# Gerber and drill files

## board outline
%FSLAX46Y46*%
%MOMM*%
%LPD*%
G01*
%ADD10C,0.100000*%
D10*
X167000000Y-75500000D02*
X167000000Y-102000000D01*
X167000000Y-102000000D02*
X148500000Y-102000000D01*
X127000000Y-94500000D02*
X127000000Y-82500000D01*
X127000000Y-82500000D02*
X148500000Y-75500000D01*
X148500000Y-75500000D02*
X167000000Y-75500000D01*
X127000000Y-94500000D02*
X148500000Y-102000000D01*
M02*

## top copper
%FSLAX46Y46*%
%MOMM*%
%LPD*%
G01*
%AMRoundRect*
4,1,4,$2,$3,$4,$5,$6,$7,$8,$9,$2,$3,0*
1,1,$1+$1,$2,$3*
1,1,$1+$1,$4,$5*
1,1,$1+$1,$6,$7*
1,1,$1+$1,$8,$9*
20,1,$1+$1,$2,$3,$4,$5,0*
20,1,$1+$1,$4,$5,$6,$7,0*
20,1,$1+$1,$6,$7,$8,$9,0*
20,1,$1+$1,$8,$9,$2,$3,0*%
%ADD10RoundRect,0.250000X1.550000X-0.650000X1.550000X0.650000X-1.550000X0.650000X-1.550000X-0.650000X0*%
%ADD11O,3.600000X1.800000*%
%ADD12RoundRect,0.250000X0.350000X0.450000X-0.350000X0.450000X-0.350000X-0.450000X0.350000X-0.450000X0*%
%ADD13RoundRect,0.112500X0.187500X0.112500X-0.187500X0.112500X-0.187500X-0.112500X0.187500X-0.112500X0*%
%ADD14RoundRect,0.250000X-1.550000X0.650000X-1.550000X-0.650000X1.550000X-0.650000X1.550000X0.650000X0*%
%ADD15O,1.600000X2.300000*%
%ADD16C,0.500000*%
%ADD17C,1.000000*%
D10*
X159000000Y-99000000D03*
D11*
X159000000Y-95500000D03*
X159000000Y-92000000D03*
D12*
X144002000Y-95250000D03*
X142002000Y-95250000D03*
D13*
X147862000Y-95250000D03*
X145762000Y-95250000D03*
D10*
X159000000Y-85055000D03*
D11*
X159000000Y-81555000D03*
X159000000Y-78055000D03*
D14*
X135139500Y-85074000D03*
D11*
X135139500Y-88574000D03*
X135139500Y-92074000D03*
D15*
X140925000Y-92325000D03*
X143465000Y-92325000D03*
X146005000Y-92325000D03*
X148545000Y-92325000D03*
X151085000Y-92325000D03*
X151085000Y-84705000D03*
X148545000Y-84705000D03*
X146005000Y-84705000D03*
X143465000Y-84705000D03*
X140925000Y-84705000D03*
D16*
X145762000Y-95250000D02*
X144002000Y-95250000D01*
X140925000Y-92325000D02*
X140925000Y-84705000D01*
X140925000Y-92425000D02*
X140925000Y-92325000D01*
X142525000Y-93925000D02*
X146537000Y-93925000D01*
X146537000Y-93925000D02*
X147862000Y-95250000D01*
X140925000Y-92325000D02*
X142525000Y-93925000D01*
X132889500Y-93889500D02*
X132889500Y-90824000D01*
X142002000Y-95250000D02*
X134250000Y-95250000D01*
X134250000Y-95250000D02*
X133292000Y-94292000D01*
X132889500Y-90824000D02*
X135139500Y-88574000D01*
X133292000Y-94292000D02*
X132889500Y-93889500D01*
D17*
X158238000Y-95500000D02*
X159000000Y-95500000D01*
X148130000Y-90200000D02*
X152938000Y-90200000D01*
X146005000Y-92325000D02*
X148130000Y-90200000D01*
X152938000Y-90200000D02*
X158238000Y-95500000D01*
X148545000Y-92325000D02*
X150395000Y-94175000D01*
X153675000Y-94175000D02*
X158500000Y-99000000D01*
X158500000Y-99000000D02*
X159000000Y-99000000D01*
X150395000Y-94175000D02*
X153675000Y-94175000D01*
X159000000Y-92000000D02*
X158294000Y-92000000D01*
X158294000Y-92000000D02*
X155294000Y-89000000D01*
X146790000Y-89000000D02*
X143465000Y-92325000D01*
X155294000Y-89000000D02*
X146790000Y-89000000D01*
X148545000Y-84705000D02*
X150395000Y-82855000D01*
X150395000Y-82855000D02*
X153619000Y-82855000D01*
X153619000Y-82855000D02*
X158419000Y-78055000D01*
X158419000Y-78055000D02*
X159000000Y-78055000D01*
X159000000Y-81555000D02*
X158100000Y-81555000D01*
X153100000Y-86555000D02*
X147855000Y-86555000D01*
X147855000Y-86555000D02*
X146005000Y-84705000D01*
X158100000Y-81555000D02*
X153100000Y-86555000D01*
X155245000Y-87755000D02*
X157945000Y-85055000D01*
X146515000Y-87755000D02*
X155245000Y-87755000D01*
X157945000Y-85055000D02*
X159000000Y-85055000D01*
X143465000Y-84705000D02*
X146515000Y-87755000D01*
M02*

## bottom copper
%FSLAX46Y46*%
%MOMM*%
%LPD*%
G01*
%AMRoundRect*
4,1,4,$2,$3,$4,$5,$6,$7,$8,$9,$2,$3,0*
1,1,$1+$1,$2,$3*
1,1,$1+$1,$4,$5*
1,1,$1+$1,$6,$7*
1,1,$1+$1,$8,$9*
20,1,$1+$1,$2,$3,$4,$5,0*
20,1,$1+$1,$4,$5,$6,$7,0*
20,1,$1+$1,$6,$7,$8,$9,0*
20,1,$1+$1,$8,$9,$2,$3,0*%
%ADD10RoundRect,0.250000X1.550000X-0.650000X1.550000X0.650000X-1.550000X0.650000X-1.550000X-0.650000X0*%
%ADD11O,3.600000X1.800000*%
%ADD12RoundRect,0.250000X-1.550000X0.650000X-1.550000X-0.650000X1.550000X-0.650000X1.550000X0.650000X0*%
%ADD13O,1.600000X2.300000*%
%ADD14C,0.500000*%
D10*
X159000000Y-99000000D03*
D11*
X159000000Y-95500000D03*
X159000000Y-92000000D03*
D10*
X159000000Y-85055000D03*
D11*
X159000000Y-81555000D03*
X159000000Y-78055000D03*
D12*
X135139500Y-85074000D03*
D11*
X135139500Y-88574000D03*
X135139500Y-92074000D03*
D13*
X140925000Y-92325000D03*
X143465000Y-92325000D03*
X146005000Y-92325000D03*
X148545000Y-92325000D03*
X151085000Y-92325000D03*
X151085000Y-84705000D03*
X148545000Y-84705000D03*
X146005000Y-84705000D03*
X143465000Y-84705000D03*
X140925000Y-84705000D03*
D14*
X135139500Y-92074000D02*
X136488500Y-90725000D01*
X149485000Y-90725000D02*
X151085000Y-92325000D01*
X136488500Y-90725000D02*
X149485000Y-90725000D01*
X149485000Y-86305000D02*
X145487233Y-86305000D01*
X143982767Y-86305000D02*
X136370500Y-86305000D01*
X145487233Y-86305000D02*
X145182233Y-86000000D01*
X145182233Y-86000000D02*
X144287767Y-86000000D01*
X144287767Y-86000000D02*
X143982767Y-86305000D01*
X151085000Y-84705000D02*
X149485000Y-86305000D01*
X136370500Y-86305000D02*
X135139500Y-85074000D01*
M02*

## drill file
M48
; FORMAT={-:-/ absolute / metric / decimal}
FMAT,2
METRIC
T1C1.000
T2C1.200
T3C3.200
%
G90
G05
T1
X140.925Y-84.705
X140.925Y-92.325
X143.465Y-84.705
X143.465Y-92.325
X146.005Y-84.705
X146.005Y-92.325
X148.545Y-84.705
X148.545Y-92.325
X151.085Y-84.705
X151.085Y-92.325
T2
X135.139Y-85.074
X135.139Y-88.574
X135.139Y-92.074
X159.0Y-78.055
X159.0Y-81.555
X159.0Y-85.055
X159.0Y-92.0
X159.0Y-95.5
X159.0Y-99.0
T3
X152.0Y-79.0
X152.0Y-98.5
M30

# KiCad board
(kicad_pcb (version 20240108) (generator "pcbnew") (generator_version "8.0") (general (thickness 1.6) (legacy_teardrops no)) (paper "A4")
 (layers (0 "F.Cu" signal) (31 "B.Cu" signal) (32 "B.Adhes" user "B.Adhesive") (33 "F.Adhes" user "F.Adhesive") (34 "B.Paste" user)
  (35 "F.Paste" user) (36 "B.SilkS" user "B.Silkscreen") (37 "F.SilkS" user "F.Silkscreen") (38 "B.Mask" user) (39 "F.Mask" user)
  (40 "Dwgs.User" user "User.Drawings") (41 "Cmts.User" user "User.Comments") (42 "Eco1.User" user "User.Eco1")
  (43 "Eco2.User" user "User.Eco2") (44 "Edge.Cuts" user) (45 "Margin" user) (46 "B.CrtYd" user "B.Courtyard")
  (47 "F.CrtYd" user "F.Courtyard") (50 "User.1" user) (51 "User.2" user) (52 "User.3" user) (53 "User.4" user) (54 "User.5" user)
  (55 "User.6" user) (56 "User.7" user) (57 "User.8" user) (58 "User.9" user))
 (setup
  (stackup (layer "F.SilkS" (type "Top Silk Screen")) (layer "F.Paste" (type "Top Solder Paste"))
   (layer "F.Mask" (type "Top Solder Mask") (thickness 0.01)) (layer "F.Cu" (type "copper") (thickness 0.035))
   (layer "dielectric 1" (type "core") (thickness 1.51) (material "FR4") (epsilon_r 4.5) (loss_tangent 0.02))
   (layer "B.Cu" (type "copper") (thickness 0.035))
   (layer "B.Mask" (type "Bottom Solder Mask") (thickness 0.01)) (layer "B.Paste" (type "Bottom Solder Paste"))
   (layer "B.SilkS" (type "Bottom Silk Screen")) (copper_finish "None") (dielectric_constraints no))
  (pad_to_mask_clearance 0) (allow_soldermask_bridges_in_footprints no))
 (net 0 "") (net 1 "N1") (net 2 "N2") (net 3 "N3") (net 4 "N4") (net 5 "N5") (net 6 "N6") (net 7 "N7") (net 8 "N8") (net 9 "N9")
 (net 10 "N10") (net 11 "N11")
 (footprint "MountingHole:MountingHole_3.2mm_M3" (layer "F.Cu") (at 152 98.5)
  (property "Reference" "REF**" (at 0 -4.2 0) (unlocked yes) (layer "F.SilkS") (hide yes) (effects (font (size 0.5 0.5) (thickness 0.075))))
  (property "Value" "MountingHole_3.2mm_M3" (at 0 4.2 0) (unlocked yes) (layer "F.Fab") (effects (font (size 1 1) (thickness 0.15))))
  (pad "" np_thru_hole circle (at 0 0) (size 3.2 3.2) (drill 3.2) (layers "*.Cu" "*.Mask")))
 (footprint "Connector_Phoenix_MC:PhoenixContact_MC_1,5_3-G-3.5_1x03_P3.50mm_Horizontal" (layer "F.Cu") (at 159 99 90)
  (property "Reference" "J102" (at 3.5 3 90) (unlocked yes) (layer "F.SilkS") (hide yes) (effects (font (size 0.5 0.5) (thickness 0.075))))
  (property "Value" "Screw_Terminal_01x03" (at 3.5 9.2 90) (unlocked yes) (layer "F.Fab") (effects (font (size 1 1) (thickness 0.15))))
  (pad "1" thru_hole roundrect (at 0 0 90) (size 1.8 3.6) (drill 1.2) (layers "*.Cu" "*.Mask") (remove_unused_layers no)
   (roundrect_rratio 0.138889) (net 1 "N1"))
  (pad "2" thru_hole oval (at 3.5 0 90) (size 1.8 3.6) (drill 1.2) (layers "*.Cu" "*.Mask") (remove_unused_layers no) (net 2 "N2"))
  (pad "3" thru_hole oval (at 7 0 90) (size 1.8 3.6) (drill 1.2) (layers "*.Cu" "*.Mask") (remove_unused_layers no) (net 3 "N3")))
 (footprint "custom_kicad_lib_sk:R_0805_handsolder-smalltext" (layer "F.Cu") (at 143.002 95.25 180)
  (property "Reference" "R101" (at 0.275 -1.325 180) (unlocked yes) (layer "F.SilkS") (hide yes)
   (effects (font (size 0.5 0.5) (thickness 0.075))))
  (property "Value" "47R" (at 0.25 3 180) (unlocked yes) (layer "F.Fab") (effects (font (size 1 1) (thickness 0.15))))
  (pad "1" smd roundrect (at -1 0 180) (size 1.2 1.4) (layers "F.Cu" "F.Paste" "F.Mask") (roundrect_rratio 0.208333) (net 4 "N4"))
  (pad "2" smd roundrect (at 1 0 180) (size 1.2 1.4) (layers "F.Cu" "F.Paste" "F.Mask") (roundrect_rratio 0.208333) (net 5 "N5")))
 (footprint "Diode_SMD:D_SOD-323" (layer "F.Cu") (at 146.812 95.25 180)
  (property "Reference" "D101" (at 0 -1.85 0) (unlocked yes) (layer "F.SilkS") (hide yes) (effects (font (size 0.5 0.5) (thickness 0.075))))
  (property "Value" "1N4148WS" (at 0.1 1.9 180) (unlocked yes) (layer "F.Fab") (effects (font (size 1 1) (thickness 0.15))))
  (pad "1" smd roundrect (at -1.05 0 180) (size 0.6 0.45) (layers "F.Cu" "F.Paste" "F.Mask") (roundrect_rratio 0.25) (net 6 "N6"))
  (pad "2" smd roundrect (at 1.05 0 180) (size 0.6 0.45) (layers "F.Cu" "F.Paste" "F.Mask") (roundrect_rratio 0.25) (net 4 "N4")))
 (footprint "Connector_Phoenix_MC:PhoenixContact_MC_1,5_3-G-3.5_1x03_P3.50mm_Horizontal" (layer "F.Cu") (at 159 85.055 90)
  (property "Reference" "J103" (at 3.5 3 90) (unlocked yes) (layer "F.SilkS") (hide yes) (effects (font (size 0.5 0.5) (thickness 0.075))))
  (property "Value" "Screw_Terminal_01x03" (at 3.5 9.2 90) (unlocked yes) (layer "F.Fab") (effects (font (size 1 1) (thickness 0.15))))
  (pad "1" thru_hole roundrect (at 0 0 90) (size 1.8 3.6) (drill 1.2) (layers "*.Cu" "*.Mask") (remove_unused_layers no)
   (roundrect_rratio 0.138889) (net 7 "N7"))
  (pad "2" thru_hole oval (at 3.5 0 90) (size 1.8 3.6) (drill 1.2) (layers "*.Cu" "*.Mask") (remove_unused_layers no) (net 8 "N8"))
  (pad "3" thru_hole oval (at 7 0 90) (size 1.8 3.6) (drill 1.2) (layers "*.Cu" "*.Mask") (remove_unused_layers no) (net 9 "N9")))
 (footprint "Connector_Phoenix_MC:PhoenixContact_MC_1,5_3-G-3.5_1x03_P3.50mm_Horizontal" (layer "F.Cu") (at 135.1395 85.074 -90)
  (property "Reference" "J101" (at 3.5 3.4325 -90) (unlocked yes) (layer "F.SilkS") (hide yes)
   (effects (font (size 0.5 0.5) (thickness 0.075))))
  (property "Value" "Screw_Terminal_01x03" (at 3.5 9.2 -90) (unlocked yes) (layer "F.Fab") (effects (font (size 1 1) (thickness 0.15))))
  (pad "1" thru_hole roundrect (at 0 0 270) (size 1.8 3.6) (drill 1.2) (layers "*.Cu" "*.Mask") (remove_unused_layers no)
   (roundrect_rratio 0.138889) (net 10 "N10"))
  (pad "2" thru_hole oval (at 3.5 0 270) (size 1.8 3.6) (drill 1.2) (layers "*.Cu" "*.Mask") (remove_unused_layers no) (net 5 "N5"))
  (pad "3" thru_hole oval (at 7 0 270) (size 1.8 3.6) (drill 1.2) (layers "*.Cu" "*.Mask") (remove_unused_layers no) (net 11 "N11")))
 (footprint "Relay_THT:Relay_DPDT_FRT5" (layer "F.Cu") (at 140.925 92.325 90)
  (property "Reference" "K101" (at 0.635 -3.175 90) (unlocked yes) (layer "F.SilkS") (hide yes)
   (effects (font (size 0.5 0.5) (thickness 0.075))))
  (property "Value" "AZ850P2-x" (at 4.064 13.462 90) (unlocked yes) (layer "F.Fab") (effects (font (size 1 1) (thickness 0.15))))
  (pad "1" thru_hole oval (at 0 0 90) (size 2.3 1.6) (drill 1) (layers "*.Cu" "*.Mask") (remove_unused_layers no) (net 6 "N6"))
  (pad "2" thru_hole oval (at 0 2.54 90) (size 2.3 1.6) (drill 1) (layers "*.Cu" "*.Mask") (remove_unused_layers no) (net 3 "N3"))
  (pad "3" thru_hole oval (at 0 5.08 90) (size 2.3 1.6) (drill 1) (layers "*.Cu" "*.Mask") (remove_unused_layers no) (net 2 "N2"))
  (pad "4" thru_hole oval (at 0 7.62 90) (size 2.3 1.6) (drill 1) (layers "*.Cu" "*.Mask") (remove_unused_layers no) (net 1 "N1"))
  (pad "5" thru_hole oval (at 0 10.16 90) (size 2.3 1.6) (drill 1) (layers "*.Cu" "*.Mask") (remove_unused_layers no) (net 11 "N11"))
  (pad "6" thru_hole oval (at 7.62 10.16 90) (size 2.3 1.6) (drill 1) (layers "*.Cu" "*.Mask") (remove_unused_layers no) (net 10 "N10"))
  (pad "7" thru_hole oval (at 7.62 7.62 90) (size 2.3 1.6) (drill 1) (layers "*.Cu" "*.Mask") (remove_unused_layers no) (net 9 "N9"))
  (pad "8" thru_hole oval (at 7.62 5.08 90) (size 2.3 1.6) (drill 1) (layers "*.Cu" "*.Mask") (remove_unused_layers no) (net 8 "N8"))
  (pad "9" thru_hole oval (at 7.62 2.54 90) (size 2.3 1.6) (drill 1) (layers "*.Cu" "*.Mask") (remove_unused_layers no) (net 7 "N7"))
  (pad "10" thru_hole oval (at 7.62 0 90) (size 2.3 1.6) (drill 1) (layers "*.Cu" "*.Mask") (remove_unused_layers no) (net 6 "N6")))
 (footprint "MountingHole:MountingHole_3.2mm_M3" (layer "F.Cu") (at 152 79)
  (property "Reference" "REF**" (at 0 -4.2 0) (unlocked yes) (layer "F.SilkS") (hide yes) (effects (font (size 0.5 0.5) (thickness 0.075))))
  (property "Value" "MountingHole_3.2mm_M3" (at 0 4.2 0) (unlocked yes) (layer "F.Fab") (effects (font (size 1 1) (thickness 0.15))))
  (pad "" np_thru_hole circle (at 0 0) (size 3.2 3.2) (drill 3.2) (layers "F&B.Cu" "*.Mask")))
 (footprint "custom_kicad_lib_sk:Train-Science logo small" (layer "B.Cu") (at 160 89 90)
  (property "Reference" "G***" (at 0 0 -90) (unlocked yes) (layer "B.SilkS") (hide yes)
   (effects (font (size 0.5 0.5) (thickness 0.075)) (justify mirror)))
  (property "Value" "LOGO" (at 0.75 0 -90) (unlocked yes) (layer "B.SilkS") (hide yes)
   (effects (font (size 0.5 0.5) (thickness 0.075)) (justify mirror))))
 (gr_line (start 167 75.5) (end 167 102) (stroke (width 0.1) (type default)) (layer "Edge.Cuts"))
 (gr_line (start 167 102) (end 148.5 102) (stroke (width 0.1) (type default)) (layer "Edge.Cuts"))
 (gr_line (start 127 94.5) (end 127 82.5) (stroke (width 0.1) (type default)) (layer "Edge.Cuts"))
 (gr_line (start 127 82.5) (end 148.5 75.5) (stroke (width 0.1) (type default)) (layer "Edge.Cuts"))
 (gr_line (start 148.5 75.5) (end 167 75.5) (stroke (width 0.1) (type default)) (layer "Edge.Cuts"))
 (gr_line (start 127 94.5) (end 148.5 102) (stroke (width 0.1) (type default)) (layer "Edge.Cuts"))
 (segment (start 145.762 95.25) (end 144.002 95.25) (width 0.5) (layer "F.Cu") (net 4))
 (segment (start 140.925 92.325) (end 140.925 84.705) (width 0.5) (layer "F.Cu") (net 6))
 (segment (start 140.925 92.425) (end 140.925 92.325) (width 0.5) (layer "F.Cu") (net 6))
 (segment (start 142.525 93.925) (end 146.537 93.925) (width 0.5) (layer "F.Cu") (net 6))
 (segment (start 146.537 93.925) (end 147.862 95.25) (width 0.5) (layer "F.Cu") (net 6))
 (segment (start 140.925 92.325) (end 142.525 93.925) (width 0.5) (layer "F.Cu") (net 6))
 (segment (start 135.1395 92.074) (end 136.4885 90.725) (width 0.5) (layer "B.Cu") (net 11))
 (segment (start 149.485 90.725) (end 151.085 92.325) (width 0.5) (layer "B.Cu") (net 11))
 (segment (start 136.4885 90.725) (end 149.485 90.725) (width 0.5) (layer "B.Cu") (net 11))
 (segment (start 149.485 86.305) (end 145.487233 86.305) (width 0.5) (layer "B.Cu") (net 10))
 (segment (start 143.982767 86.305) (end 136.3705 86.305) (width 0.5) (layer "B.Cu") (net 10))
 (segment (start 145.487233 86.305) (end 145.182233 86) (width 0.5) (layer "B.Cu") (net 10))
 (segment (start 145.182233 86) (end 144.287767 86) (width 0.5) (layer "B.Cu") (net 10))
 (segment (start 144.287767 86) (end 143.982767 86.305) (width 0.5) (layer "B.Cu") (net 10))
 (segment (start 151.085 84.705) (end 149.485 86.305) (width 0.5) (layer "B.Cu") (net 10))
 (segment (start 136.3705 86.305) (end 135.1395 85.074) (width 0.5) (layer "B.Cu") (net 10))
 (segment (start 132.8895 93.8895) (end 132.8895 90.824) (width 0.5) (layer "F.Cu") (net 5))
 (segment (start 142.002 95.25) (end 134.25 95.25) (width 0.5) (layer "F.Cu") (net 5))
 (segment (start 134.25 95.25) (end 133.292 94.292) (width 0.5) (layer "F.Cu") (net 5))
 (segment (start 132.8895 90.824) (end 135.1395 88.574) (width 0.5) (layer "F.Cu") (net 5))
 (segment (start 133.292 94.292) (end 132.8895 93.8895) (width 0.5) (layer "F.Cu") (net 5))
 (segment (start 158.238 95.5) (end 159 95.5) (width 1) (layer "F.Cu") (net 2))
 (segment (start 148.13 90.2) (end 152.938 90.2) (width 1) (layer "F.Cu") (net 2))
 (segment (start 146.005 92.325) (end 148.13 90.2) (width 1) (layer "F.Cu") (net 2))
 (segment (start 152.938 90.2) (end 158.238 95.5) (width 1) (layer "F.Cu") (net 2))
 (segment (start 148.545 92.325) (end 150.395 94.175) (width 1) (layer "F.Cu") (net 1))
 (segment (start 153.675 94.175) (end 158.5 99) (width 1) (layer "F.Cu") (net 1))
 (segment (start 158.5 99) (end 159 99) (width 1) (layer "F.Cu") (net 1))
 (segment (start 150.395 94.175) (end 153.675 94.175) (width 1) (layer "F.Cu") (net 1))
 (segment (start 159 92) (end 158.294 92) (width 1) (layer "F.Cu") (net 3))
 (segment (start 158.294 92) (end 155.294 89) (width 1) (layer "F.Cu") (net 3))
 (segment (start 146.79 89) (end 143.465 92.325) (width 1) (layer "F.Cu") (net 3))
 (segment (start 155.294 89) (end 146.79 89) (width 1) (layer "F.Cu") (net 3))
 (segment (start 148.545 84.705) (end 150.395 82.855) (width 1) (layer "F.Cu") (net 9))
 (segment (start 150.395 82.855) (end 153.619 82.855) (width 1) (layer "F.Cu") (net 9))
 (segment (start 153.619 82.855) (end 158.419 78.055) (width 1) (layer "F.Cu") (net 9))
 (segment (start 158.419 78.055) (end 159 78.055) (width 1) (layer "F.Cu") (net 9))
 (segment (start 159 81.555) (end 158.1 81.555) (width 1) (layer "F.Cu") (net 8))
 (segment (start 153.1 86.555) (end 147.855 86.555) (width 1) (layer "F.Cu") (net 8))
 (segment (start 147.855 86.555) (end 146.005 84.705) (width 1) (layer "F.Cu") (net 8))
 (segment (start 158.1 81.555) (end 153.1 86.555) (width 1) (layer "F.Cu") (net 8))
 (segment (start 155.245 87.755) (end 157.945 85.055) (width 1) (layer "F.Cu") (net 7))
 (segment (start 146.515 87.755) (end 155.245 87.755) (width 1) (layer "F.Cu") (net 7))
 (segment (start 157.945 85.055) (end 159 85.055) (width 1) (layer "F.Cu") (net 7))
 (segment (start 143.465 84.705) (end 146.515 87.755) (width 1) (layer "F.Cu") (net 7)))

